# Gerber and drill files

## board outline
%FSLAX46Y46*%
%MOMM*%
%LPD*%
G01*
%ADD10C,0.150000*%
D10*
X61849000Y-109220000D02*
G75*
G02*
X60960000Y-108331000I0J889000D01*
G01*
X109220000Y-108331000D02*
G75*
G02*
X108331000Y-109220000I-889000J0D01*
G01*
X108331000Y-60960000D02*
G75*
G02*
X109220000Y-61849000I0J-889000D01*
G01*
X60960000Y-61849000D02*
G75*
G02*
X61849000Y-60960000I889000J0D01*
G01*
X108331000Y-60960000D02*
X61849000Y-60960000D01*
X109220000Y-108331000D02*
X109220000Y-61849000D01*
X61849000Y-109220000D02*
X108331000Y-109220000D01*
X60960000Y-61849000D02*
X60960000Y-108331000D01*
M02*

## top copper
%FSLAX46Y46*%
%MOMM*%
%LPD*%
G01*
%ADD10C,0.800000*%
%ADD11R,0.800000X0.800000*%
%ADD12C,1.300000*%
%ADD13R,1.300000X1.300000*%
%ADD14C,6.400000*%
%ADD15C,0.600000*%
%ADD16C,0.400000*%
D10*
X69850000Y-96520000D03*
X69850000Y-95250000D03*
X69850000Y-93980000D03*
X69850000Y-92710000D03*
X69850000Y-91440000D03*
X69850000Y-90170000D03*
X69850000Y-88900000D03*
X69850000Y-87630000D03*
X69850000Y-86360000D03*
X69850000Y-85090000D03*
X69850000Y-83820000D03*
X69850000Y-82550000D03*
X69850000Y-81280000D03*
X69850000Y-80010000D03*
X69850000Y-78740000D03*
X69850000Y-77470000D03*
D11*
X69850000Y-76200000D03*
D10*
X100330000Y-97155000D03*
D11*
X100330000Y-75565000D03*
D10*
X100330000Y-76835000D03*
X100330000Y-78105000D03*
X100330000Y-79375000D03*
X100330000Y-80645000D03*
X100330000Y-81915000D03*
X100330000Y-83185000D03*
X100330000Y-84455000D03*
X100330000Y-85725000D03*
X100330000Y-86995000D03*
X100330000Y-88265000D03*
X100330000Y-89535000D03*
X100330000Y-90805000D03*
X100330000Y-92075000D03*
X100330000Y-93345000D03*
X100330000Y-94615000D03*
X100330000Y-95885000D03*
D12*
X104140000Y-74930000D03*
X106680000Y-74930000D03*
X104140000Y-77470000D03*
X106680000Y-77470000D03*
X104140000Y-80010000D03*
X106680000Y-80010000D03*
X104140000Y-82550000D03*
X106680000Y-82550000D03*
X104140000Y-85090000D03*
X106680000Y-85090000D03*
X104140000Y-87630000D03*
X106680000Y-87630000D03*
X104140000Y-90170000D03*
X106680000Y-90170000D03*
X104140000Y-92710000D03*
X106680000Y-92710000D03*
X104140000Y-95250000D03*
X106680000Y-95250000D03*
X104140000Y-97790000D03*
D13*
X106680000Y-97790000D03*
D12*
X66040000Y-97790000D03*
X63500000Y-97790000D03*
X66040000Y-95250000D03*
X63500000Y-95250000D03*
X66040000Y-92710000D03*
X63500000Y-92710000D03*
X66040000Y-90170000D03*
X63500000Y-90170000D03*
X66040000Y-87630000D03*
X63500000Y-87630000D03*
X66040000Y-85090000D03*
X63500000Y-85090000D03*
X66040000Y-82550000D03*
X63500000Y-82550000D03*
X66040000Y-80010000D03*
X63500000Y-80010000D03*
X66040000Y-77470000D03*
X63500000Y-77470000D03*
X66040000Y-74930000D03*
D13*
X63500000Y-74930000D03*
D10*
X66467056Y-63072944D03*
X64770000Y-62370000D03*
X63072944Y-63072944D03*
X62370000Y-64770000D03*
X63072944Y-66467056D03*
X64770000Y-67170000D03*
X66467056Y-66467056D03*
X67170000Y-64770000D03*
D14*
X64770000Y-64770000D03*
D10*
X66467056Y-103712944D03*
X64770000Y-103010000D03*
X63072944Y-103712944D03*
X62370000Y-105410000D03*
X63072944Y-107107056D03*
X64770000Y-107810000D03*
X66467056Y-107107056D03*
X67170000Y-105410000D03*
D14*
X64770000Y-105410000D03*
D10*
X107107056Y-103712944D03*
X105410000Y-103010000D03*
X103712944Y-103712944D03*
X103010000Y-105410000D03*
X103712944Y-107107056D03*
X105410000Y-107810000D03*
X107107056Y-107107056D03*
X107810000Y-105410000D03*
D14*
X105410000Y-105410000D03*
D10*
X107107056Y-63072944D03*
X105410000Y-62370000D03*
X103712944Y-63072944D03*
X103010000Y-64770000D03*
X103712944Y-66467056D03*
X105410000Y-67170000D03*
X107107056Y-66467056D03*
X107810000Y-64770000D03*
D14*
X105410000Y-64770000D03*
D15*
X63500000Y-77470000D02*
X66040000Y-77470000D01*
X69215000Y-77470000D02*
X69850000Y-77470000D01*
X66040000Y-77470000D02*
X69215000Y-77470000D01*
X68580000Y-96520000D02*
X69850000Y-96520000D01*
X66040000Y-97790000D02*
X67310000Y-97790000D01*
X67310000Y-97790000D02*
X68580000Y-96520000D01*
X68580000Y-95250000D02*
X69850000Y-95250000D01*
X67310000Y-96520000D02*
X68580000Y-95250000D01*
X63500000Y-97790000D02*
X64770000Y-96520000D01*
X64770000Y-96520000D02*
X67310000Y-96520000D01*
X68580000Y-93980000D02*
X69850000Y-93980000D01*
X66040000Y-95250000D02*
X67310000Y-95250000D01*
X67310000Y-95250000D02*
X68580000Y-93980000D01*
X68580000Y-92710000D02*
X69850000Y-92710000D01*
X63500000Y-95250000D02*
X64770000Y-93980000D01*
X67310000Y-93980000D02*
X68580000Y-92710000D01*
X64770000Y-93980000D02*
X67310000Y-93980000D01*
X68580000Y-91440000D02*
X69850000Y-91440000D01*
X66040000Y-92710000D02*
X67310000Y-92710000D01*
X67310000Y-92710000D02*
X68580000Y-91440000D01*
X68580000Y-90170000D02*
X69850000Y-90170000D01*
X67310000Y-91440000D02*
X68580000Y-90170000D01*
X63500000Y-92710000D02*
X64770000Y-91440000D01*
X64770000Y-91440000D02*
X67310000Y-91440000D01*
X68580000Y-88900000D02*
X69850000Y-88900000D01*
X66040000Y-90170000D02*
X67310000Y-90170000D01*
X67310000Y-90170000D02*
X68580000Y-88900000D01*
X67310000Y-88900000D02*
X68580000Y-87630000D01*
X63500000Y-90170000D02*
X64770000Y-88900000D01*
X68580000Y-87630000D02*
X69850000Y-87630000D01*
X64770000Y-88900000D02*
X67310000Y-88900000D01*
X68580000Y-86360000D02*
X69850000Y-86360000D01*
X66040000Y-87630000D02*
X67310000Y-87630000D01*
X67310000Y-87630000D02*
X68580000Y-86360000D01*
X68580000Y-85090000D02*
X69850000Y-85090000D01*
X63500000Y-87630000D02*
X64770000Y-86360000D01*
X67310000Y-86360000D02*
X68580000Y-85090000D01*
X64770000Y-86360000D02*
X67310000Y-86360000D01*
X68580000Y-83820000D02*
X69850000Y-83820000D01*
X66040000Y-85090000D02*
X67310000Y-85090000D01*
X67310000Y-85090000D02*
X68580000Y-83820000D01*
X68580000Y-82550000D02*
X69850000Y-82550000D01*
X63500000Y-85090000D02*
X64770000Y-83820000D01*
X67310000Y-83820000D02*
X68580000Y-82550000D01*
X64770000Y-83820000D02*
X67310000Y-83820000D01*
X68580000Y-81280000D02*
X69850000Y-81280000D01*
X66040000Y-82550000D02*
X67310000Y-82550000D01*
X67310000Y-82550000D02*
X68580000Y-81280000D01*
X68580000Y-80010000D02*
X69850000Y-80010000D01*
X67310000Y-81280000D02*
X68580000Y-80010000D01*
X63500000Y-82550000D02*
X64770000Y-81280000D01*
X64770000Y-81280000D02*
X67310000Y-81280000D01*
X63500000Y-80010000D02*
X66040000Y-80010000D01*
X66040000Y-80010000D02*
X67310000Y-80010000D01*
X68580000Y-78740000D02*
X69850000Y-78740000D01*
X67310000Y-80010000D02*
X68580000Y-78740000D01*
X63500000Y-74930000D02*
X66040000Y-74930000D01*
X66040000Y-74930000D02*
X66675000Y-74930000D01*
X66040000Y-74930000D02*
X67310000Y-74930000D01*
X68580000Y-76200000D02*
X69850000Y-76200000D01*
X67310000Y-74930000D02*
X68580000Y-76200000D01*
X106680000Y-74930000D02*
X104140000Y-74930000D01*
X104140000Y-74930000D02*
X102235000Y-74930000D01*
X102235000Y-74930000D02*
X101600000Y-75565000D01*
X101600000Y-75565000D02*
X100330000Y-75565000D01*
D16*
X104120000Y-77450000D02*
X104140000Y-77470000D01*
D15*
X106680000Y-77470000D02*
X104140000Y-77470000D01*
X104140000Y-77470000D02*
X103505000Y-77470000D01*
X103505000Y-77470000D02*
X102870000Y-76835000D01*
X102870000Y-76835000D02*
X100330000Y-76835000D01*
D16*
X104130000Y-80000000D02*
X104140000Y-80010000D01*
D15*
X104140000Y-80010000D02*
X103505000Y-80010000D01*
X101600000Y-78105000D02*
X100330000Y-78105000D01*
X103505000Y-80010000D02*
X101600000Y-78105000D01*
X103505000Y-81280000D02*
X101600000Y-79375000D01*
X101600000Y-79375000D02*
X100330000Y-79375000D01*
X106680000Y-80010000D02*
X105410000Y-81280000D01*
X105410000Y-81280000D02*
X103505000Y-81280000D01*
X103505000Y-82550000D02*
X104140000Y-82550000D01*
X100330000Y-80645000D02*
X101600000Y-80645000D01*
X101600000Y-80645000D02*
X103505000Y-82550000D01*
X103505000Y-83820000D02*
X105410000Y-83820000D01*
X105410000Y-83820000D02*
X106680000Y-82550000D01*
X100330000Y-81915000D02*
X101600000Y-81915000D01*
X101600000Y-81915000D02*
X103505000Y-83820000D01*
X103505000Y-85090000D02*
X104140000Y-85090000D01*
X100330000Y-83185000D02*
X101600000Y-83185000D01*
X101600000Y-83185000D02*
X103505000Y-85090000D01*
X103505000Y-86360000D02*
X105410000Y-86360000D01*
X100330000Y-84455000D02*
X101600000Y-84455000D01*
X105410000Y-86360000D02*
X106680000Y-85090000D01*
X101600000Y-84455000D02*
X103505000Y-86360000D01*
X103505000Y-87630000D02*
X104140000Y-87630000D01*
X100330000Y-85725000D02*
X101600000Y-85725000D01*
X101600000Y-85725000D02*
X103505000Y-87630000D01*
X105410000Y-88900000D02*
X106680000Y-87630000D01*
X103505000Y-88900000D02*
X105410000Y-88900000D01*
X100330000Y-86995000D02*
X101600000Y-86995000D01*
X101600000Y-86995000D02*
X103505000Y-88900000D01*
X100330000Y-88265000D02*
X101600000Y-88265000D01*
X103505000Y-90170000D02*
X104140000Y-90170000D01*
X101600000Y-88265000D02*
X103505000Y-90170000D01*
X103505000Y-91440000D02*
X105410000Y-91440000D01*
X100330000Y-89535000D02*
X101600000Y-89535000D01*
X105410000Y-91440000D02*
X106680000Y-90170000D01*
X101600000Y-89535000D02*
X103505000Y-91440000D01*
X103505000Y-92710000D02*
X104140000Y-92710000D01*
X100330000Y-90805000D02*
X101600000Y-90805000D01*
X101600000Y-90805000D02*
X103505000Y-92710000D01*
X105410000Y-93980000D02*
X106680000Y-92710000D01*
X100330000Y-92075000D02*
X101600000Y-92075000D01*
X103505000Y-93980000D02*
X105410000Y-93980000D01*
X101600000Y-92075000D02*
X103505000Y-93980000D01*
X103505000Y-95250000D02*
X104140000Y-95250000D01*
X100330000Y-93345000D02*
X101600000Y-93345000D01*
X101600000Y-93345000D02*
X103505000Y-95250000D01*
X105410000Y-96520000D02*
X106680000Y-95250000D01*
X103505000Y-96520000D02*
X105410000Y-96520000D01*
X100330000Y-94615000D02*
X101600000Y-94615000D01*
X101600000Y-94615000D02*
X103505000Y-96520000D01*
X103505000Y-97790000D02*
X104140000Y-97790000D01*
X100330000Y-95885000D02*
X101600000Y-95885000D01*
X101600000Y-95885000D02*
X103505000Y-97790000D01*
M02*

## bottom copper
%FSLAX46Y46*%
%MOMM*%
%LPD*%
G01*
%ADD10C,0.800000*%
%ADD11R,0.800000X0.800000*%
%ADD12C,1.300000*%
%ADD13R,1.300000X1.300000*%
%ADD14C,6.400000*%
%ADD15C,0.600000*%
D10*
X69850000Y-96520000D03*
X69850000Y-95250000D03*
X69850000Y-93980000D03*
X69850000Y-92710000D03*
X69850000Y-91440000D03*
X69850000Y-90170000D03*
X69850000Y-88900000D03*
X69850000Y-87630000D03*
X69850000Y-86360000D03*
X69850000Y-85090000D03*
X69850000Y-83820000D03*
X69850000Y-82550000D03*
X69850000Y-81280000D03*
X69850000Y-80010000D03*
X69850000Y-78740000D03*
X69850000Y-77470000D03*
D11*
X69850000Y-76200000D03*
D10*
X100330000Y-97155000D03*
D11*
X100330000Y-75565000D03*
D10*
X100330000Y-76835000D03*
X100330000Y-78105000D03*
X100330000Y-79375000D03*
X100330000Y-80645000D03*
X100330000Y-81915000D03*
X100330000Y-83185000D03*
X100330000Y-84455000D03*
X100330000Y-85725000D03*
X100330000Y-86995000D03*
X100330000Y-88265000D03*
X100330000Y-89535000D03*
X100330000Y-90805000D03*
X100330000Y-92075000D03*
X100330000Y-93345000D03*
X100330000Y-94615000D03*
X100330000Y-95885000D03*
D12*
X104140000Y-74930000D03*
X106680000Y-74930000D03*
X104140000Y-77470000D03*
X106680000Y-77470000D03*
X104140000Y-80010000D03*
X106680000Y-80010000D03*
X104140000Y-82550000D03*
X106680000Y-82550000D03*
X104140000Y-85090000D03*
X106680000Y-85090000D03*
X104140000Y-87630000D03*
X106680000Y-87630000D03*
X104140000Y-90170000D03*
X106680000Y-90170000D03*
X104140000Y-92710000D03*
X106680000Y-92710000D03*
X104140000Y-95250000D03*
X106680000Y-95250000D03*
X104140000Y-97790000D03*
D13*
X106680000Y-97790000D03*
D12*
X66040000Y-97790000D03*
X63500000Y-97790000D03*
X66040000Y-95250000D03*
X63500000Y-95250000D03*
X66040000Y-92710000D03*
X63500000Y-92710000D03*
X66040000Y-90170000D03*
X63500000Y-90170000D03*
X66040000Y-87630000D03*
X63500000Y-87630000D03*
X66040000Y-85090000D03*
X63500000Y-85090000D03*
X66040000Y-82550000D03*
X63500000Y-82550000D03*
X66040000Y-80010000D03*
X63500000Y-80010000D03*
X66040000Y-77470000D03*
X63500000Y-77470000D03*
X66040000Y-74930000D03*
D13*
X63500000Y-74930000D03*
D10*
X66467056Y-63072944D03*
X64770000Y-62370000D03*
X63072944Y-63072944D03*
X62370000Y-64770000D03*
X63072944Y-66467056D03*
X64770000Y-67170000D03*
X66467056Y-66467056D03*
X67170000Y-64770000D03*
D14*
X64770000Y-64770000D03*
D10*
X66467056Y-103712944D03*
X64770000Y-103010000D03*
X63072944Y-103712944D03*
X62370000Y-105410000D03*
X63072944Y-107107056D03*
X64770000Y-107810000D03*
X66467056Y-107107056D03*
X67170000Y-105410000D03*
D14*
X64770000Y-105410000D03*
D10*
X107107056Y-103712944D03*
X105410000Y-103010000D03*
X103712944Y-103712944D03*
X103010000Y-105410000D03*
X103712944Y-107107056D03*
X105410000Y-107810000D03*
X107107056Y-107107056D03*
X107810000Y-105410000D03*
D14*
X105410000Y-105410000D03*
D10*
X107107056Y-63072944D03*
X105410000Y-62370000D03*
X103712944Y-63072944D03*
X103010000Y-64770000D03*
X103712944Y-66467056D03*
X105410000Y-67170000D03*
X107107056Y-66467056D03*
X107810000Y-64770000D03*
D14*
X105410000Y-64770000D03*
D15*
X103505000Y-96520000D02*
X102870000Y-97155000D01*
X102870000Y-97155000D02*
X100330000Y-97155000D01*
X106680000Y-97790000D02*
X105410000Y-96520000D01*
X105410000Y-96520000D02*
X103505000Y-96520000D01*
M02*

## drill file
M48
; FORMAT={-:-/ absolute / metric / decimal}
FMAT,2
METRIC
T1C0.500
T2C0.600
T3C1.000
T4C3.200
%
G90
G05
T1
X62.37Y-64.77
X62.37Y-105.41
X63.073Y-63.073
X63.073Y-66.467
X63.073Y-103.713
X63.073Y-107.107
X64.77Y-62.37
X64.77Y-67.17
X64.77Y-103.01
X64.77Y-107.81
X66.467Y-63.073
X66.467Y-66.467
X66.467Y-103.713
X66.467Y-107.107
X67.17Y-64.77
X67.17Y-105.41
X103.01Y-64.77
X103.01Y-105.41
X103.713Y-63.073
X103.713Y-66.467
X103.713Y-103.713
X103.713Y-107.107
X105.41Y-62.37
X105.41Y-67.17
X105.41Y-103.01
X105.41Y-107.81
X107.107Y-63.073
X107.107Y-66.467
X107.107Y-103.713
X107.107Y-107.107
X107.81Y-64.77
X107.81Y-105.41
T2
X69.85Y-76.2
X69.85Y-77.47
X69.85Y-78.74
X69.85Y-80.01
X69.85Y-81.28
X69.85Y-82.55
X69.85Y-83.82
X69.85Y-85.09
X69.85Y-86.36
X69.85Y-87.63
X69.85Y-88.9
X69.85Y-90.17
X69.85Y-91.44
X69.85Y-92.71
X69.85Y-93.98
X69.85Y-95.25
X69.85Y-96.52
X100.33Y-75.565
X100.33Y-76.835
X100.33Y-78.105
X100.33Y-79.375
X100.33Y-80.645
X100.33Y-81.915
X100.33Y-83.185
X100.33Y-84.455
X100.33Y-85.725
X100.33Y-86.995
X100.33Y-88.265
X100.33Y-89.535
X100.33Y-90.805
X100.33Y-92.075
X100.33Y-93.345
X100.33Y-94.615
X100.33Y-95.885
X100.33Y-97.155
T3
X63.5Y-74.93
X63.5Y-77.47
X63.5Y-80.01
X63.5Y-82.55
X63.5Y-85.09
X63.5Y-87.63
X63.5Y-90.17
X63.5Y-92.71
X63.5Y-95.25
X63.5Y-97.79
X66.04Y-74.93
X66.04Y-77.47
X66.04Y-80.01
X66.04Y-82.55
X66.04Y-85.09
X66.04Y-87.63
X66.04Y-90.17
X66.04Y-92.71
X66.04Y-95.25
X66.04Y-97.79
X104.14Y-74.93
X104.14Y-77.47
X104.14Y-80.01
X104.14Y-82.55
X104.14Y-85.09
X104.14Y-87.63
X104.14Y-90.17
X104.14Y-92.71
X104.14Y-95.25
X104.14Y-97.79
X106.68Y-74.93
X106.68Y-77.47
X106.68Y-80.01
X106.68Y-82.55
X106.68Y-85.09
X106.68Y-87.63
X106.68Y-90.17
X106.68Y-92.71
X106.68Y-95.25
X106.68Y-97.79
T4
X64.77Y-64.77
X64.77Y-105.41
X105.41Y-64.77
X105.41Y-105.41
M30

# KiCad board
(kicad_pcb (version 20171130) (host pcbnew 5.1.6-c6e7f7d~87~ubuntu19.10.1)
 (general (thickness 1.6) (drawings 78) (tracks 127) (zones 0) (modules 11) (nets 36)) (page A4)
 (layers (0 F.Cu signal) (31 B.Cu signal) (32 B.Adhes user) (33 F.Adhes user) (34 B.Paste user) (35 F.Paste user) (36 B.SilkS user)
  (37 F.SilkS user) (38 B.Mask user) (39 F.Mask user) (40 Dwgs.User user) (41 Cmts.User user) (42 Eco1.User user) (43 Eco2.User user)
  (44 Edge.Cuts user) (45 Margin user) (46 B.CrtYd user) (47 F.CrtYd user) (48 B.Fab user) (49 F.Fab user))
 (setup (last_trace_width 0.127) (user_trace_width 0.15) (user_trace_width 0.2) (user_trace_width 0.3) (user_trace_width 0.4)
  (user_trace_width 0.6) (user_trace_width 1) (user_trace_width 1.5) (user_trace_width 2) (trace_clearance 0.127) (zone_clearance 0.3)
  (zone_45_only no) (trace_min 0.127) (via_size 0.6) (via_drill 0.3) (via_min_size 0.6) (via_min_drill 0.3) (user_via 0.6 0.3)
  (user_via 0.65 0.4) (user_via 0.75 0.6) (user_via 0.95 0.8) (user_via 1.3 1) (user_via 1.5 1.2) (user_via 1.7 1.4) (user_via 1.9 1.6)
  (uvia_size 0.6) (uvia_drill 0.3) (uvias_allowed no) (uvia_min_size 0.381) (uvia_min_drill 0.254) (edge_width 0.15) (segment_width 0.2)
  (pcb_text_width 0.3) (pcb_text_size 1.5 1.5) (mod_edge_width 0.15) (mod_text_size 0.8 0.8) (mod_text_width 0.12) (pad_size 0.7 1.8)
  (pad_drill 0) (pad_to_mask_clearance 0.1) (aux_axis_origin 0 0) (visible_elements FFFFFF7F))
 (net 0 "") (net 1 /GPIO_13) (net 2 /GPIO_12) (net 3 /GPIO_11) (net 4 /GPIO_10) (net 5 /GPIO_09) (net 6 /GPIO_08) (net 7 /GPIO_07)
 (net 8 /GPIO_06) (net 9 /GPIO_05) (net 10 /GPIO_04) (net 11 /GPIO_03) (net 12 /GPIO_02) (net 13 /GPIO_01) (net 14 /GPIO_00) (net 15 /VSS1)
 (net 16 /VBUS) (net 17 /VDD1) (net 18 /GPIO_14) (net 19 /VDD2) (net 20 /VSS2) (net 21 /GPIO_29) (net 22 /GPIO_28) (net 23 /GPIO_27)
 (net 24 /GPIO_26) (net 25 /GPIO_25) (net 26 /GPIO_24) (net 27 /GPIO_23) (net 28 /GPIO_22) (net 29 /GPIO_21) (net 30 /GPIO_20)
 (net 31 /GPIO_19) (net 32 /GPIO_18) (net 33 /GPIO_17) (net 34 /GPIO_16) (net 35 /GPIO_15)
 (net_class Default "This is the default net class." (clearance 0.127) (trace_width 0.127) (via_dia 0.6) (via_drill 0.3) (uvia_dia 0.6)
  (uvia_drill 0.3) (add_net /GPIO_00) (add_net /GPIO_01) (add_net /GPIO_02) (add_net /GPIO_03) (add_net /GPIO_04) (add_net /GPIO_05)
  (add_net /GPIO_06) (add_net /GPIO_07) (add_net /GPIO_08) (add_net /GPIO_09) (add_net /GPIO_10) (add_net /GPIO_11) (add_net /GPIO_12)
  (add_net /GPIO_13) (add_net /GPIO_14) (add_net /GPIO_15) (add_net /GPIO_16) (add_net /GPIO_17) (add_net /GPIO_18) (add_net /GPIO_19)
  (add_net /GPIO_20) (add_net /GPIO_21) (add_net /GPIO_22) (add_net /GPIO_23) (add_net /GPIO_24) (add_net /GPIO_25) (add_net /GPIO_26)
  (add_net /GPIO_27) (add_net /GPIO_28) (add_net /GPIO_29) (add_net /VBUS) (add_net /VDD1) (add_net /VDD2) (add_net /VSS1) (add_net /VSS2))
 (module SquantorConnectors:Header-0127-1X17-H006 (layer F.Cu) (at 69.85 86.36 270)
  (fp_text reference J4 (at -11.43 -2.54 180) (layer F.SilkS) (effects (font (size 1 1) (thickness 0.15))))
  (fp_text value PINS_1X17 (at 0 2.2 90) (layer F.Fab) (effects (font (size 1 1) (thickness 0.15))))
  (pad 17 thru_hole circle (at 10.16 0 270) (size 0.8 0.8) (drill 0.6) (layers *.Cu *.Mask) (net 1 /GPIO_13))
  (pad 16 thru_hole circle (at 8.89 0 270) (size 0.8 0.8) (drill 0.6) (layers *.Cu *.Mask) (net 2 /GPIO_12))
  (pad 15 thru_hole circle (at 7.62 0 270) (size 0.8 0.8) (drill 0.6) (layers *.Cu *.Mask) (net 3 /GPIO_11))
  (pad 14 thru_hole circle (at 6.35 0 270) (size 0.8 0.8) (drill 0.6) (layers *.Cu *.Mask) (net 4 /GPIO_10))
  (pad 13 thru_hole circle (at 5.08 0 270) (size 0.8 0.8) (drill 0.6) (layers *.Cu *.Mask) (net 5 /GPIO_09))
  (pad 12 thru_hole circle (at 3.81 0 270) (size 0.8 0.8) (drill 0.6) (layers *.Cu *.Mask) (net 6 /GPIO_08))
  (pad 11 thru_hole circle (at 2.54 0 270) (size 0.8 0.8) (drill 0.6) (layers *.Cu *.Mask) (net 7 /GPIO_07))
  (pad 10 thru_hole circle (at 1.27 0 270) (size 0.8 0.8) (drill 0.6) (layers *.Cu *.Mask) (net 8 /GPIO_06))
  (pad 9 thru_hole circle (at 0 0 270) (size 0.8 0.8) (drill 0.6) (layers *.Cu *.Mask) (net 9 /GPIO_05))
  (pad 8 thru_hole circle (at -1.27 0 270) (size 0.8 0.8) (drill 0.6) (layers *.Cu *.Mask) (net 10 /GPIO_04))
  (pad 7 thru_hole circle (at -2.54 0 270) (size 0.8 0.8) (drill 0.6) (layers *.Cu *.Mask) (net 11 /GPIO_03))
  (pad 6 thru_hole circle (at -3.81 0 270) (size 0.8 0.8) (drill 0.6) (layers *.Cu *.Mask) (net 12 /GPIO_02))
  (pad 5 thru_hole circle (at -5.08 0 270) (size 0.8 0.8) (drill 0.6) (layers *.Cu *.Mask) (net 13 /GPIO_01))
  (pad 4 thru_hole circle (at -6.35 0 270) (size 0.8 0.8) (drill 0.6) (layers *.Cu *.Mask) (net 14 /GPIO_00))
  (pad 3 thru_hole circle (at -7.62 0 270) (size 0.8 0.8) (drill 0.6) (layers *.Cu *.Mask) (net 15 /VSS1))
  (pad 2 thru_hole circle (at -8.89 0 270) (size 0.8 0.8) (drill 0.6) (layers *.Cu *.Mask) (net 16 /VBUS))
  (pad 1 thru_hole rect (at -10.16 0 270) (size 0.8 0.8) (drill 0.6) (layers *.Cu *.Mask) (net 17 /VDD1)))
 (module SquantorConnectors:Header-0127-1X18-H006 (layer F.Cu) (at 100.33 86.36 270)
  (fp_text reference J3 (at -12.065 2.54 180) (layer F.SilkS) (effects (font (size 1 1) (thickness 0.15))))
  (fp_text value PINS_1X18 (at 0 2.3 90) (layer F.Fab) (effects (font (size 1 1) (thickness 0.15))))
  (pad 18 thru_hole circle (at 10.795 0 270) (size 0.8 0.8) (drill 0.6) (layers *.Cu *.Mask) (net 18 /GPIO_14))
  (pad 1 thru_hole rect (at -10.795 0 270) (size 0.8 0.8) (drill 0.6) (layers *.Cu *.Mask) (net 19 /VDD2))
  (pad 2 thru_hole circle (at -9.525 0 270) (size 0.8 0.8) (drill 0.6) (layers *.Cu *.Mask) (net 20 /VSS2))
  (pad 3 thru_hole circle (at -8.255 0 270) (size 0.8 0.8) (drill 0.6) (layers *.Cu *.Mask) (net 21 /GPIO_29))
  (pad 4 thru_hole circle (at -6.985 0 270) (size 0.8 0.8) (drill 0.6) (layers *.Cu *.Mask) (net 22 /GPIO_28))
  (pad 5 thru_hole circle (at -5.715 0 270) (size 0.8 0.8) (drill 0.6) (layers *.Cu *.Mask) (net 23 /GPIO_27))
  (pad 6 thru_hole circle (at -4.445 0 270) (size 0.8 0.8) (drill 0.6) (layers *.Cu *.Mask) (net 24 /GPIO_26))
  (pad 7 thru_hole circle (at -3.175 0 270) (size 0.8 0.8) (drill 0.6) (layers *.Cu *.Mask) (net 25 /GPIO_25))
  (pad 8 thru_hole circle (at -1.905 0 270) (size 0.8 0.8) (drill 0.6) (layers *.Cu *.Mask) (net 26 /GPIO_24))
  (pad 9 thru_hole circle (at -0.635 0 270) (size 0.8 0.8) (drill 0.6) (layers *.Cu *.Mask) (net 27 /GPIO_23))
  (pad 10 thru_hole circle (at 0.635 0 270) (size 0.8 0.8) (drill 0.6) (layers *.Cu *.Mask) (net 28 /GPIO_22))
  (pad 11 thru_hole circle (at 1.905 0 270) (size 0.8 0.8) (drill 0.6) (layers *.Cu *.Mask) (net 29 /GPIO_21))
  (pad 12 thru_hole circle (at 3.175 0 270) (size 0.8 0.8) (drill 0.6) (layers *.Cu *.Mask) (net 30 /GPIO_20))
  (pad 13 thru_hole circle (at 4.445 0 270) (size 0.8 0.8) (drill 0.6) (layers *.Cu *.Mask) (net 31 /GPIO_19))
  (pad 14 thru_hole circle (at 5.715 0 270) (size 0.8 0.8) (drill 0.6) (layers *.Cu *.Mask) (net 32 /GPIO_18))
  (pad 15 thru_hole circle (at 6.985 0 270) (size 0.8 0.8) (drill 0.6) (layers *.Cu *.Mask) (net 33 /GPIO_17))
  (pad 16 thru_hole circle (at 8.255 0 270) (size 0.8 0.8) (drill 0.6) (layers *.Cu *.Mask) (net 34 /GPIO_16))
  (pad 17 thru_hole circle (at 9.525 0 270) (size 0.8 0.8) (drill 0.6) (layers *.Cu *.Mask) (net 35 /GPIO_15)))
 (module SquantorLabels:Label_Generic (layer B.Cu) (at 83.7 105.9)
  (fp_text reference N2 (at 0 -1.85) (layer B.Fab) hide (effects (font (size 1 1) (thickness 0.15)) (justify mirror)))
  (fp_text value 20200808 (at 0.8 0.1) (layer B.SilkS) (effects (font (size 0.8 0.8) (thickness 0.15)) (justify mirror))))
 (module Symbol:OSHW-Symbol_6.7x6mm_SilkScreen (layer B.Cu) (at 85.2 101.9 180)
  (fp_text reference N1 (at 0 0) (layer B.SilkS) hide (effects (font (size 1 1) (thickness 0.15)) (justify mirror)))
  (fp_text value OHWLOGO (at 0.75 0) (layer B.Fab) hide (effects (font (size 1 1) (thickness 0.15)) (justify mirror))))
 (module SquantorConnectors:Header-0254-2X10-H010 (layer F.Cu) (at 105.41 86.36 90)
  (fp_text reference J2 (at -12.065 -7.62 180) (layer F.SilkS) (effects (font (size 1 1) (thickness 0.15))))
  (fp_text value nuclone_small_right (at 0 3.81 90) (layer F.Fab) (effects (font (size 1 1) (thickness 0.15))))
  (pad 20 thru_hole circle (at 11.43 -1.27 90) (size 1.3 1.3) (drill 1) (layers *.Cu *.Mask) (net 19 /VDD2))
  (pad 19 thru_hole circle (at 11.43 1.27 90) (size 1.3 1.3) (drill 1) (layers *.Cu *.Mask) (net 19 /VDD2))
  (pad 18 thru_hole circle (at 8.89 -1.27 90) (size 1.3 1.3) (drill 1) (layers *.Cu *.Mask) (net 20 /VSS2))
  (pad 17 thru_hole circle (at 8.89 1.27 90) (size 1.3 1.3) (drill 1) (layers *.Cu *.Mask) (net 20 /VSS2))
  (pad 16 thru_hole circle (at 6.35 -1.27 90) (size 1.3 1.3) (drill 1) (layers *.Cu *.Mask) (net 21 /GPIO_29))
  (pad 15 thru_hole circle (at 6.35 1.27 90) (size 1.3 1.3) (drill 1) (layers *.Cu *.Mask) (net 22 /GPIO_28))
  (pad 14 thru_hole circle (at 3.81 -1.27 90) (size 1.3 1.3) (drill 1) (layers *.Cu *.Mask) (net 23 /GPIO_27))
  (pad 13 thru_hole circle (at 3.81 1.27 90) (size 1.3 1.3) (drill 1) (layers *.Cu *.Mask) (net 24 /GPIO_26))
  (pad 12 thru_hole circle (at 1.27 -1.27 90) (size 1.3 1.3) (drill 1) (layers *.Cu *.Mask) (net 25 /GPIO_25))
  (pad 11 thru_hole circle (at 1.27 1.27 90) (size 1.3 1.3) (drill 1) (layers *.Cu *.Mask) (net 26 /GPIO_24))
  (pad 10 thru_hole circle (at -1.27 -1.27 90) (size 1.3 1.3) (drill 1) (layers *.Cu *.Mask) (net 27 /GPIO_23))
  (pad 9 thru_hole circle (at -1.27 1.27 90) (size 1.3 1.3) (drill 1) (layers *.Cu *.Mask) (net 28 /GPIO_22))
  (pad 8 thru_hole circle (at -3.81 -1.27 90) (size 1.3 1.3) (drill 1) (layers *.Cu *.Mask) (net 29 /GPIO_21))
  (pad 7 thru_hole circle (at -3.81 1.27 90) (size 1.3 1.3) (drill 1) (layers *.Cu *.Mask) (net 30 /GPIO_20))
  (pad 6 thru_hole circle (at -6.35 -1.27 90) (size 1.3 1.3) (drill 1) (layers *.Cu *.Mask) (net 31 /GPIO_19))
  (pad 5 thru_hole circle (at -6.35 1.27 90) (size 1.3 1.3) (drill 1) (layers *.Cu *.Mask) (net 32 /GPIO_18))
  (pad 4 thru_hole circle (at -8.89 -1.27 90) (size 1.3 1.3) (drill 1) (layers *.Cu *.Mask) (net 33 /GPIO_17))
  (pad 3 thru_hole circle (at -8.89 1.27 90) (size 1.3 1.3) (drill 1) (layers *.Cu *.Mask) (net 34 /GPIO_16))
  (pad 2 thru_hole circle (at -11.43 -1.27 90) (size 1.3 1.3) (drill 1) (layers *.Cu *.Mask) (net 35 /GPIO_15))
  (pad 1 thru_hole rect (at -11.43 1.27 90) (size 1.3 1.3) (drill 1) (layers *.Cu *.Mask) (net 18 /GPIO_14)))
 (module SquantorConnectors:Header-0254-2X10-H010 (layer F.Cu) (at 64.77 86.36 270)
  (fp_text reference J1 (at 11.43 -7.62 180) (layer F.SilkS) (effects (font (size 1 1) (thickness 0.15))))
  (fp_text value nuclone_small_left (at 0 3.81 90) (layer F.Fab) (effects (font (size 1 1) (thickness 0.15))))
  (pad 20 thru_hole circle (at 11.43 -1.27 270) (size 1.3 1.3) (drill 1) (layers *.Cu *.Mask) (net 1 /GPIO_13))
  (pad 19 thru_hole circle (at 11.43 1.27 270) (size 1.3 1.3) (drill 1) (layers *.Cu *.Mask) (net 2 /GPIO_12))
  (pad 18 thru_hole circle (at 8.89 -1.27 270) (size 1.3 1.3) (drill 1) (layers *.Cu *.Mask) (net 3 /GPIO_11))
  (pad 17 thru_hole circle (at 8.89 1.27 270) (size 1.3 1.3) (drill 1) (layers *.Cu *.Mask) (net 4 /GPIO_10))
  (pad 16 thru_hole circle (at 6.35 -1.27 270) (size 1.3 1.3) (drill 1) (layers *.Cu *.Mask) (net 5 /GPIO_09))
  (pad 15 thru_hole circle (at 6.35 1.27 270) (size 1.3 1.3) (drill 1) (layers *.Cu *.Mask) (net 6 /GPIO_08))
  (pad 14 thru_hole circle (at 3.81 -1.27 270) (size 1.3 1.3) (drill 1) (layers *.Cu *.Mask) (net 7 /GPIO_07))
  (pad 13 thru_hole circle (at 3.81 1.27 270) (size 1.3 1.3) (drill 1) (layers *.Cu *.Mask) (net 8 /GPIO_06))
  (pad 12 thru_hole circle (at 1.27 -1.27 270) (size 1.3 1.3) (drill 1) (layers *.Cu *.Mask) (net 9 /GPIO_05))
  (pad 11 thru_hole circle (at 1.27 1.27 270) (size 1.3 1.3) (drill 1) (layers *.Cu *.Mask) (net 10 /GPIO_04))
  (pad 10 thru_hole circle (at -1.27 -1.27 270) (size 1.3 1.3) (drill 1) (layers *.Cu *.Mask) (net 11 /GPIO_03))
  (pad 9 thru_hole circle (at -1.27 1.27 270) (size 1.3 1.3) (drill 1) (layers *.Cu *.Mask) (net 12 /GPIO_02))
  (pad 8 thru_hole circle (at -3.81 -1.27 270) (size 1.3 1.3) (drill 1) (layers *.Cu *.Mask) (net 13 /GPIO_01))
  (pad 7 thru_hole circle (at -3.81 1.27 270) (size 1.3 1.3) (drill 1) (layers *.Cu *.Mask) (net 14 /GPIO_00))
  (pad 6 thru_hole circle (at -6.35 -1.27 270) (size 1.3 1.3) (drill 1) (layers *.Cu *.Mask) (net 15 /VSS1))
  (pad 5 thru_hole circle (at -6.35 1.27 270) (size 1.3 1.3) (drill 1) (layers *.Cu *.Mask) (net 15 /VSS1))
  (pad 4 thru_hole circle (at -8.89 -1.27 270) (size 1.3 1.3) (drill 1) (layers *.Cu *.Mask) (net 16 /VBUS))
  (pad 3 thru_hole circle (at -8.89 1.27 270) (size 1.3 1.3) (drill 1) (layers *.Cu *.Mask) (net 16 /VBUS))
  (pad 2 thru_hole circle (at -11.43 -1.27 270) (size 1.3 1.3) (drill 1) (layers *.Cu *.Mask) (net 17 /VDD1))
  (pad 1 thru_hole rect (at -11.43 1.27 270) (size 1.3 1.3) (drill 1) (layers *.Cu *.Mask) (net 17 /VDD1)))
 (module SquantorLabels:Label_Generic (layer B.Cu) (at 86 107.9 180)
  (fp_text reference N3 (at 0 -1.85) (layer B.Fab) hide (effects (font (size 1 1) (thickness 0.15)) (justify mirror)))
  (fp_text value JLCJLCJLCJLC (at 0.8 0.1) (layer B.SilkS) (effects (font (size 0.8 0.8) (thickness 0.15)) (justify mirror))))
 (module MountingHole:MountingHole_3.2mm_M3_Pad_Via (layer F.Cu) (at 64.77 64.77)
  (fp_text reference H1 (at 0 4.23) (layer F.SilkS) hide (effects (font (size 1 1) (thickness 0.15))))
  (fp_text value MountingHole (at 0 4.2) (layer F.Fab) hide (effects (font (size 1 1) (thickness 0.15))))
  (pad 1 thru_hole circle (at 1.697056 -1.697056) (size 0.8 0.8) (drill 0.5) (layers *.Cu *.Mask))
  (pad 1 thru_hole circle (at 0 -2.4) (size 0.8 0.8) (drill 0.5) (layers *.Cu *.Mask))
  (pad 1 thru_hole circle (at -1.697056 -1.697056) (size 0.8 0.8) (drill 0.5) (layers *.Cu *.Mask))
  (pad 1 thru_hole circle (at -2.4 0) (size 0.8 0.8) (drill 0.5) (layers *.Cu *.Mask))
  (pad 1 thru_hole circle (at -1.697056 1.697056) (size 0.8 0.8) (drill 0.5) (layers *.Cu *.Mask))
  (pad 1 thru_hole circle (at 0 2.4) (size 0.8 0.8) (drill 0.5) (layers *.Cu *.Mask))
  (pad 1 thru_hole circle (at 1.697056 1.697056) (size 0.8 0.8) (drill 0.5) (layers *.Cu *.Mask))
  (pad 1 thru_hole circle (at 2.4 0) (size 0.8 0.8) (drill 0.5) (layers *.Cu *.Mask))
  (pad 1 thru_hole circle (at 0 0) (size 6.4 6.4) (drill 3.2) (layers *.Cu *.Mask)))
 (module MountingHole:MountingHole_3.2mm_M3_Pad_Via (layer F.Cu) (at 64.77 105.41)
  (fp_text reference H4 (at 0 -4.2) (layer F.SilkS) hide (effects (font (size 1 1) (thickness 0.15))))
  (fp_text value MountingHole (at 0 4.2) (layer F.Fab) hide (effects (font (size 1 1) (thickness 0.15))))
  (pad 1 thru_hole circle (at 1.697056 -1.697056) (size 0.8 0.8) (drill 0.5) (layers *.Cu *.Mask))
  (pad 1 thru_hole circle (at 0 -2.4) (size 0.8 0.8) (drill 0.5) (layers *.Cu *.Mask))
  (pad 1 thru_hole circle (at -1.697056 -1.697056) (size 0.8 0.8) (drill 0.5) (layers *.Cu *.Mask))
  (pad 1 thru_hole circle (at -2.4 0) (size 0.8 0.8) (drill 0.5) (layers *.Cu *.Mask))
  (pad 1 thru_hole circle (at -1.697056 1.697056) (size 0.8 0.8) (drill 0.5) (layers *.Cu *.Mask))
  (pad 1 thru_hole circle (at 0 2.4) (size 0.8 0.8) (drill 0.5) (layers *.Cu *.Mask))
  (pad 1 thru_hole circle (at 1.697056 1.697056) (size 0.8 0.8) (drill 0.5) (layers *.Cu *.Mask))
  (pad 1 thru_hole circle (at 2.4 0) (size 0.8 0.8) (drill 0.5) (layers *.Cu *.Mask))
  (pad 1 thru_hole circle (at 0 0) (size 6.4 6.4) (drill 3.2) (layers *.Cu *.Mask)))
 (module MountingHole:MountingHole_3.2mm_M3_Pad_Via (layer F.Cu) (at 105.41 105.41)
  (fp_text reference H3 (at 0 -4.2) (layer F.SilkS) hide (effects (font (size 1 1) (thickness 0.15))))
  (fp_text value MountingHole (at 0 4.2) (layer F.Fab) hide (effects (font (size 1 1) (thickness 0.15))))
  (pad 1 thru_hole circle (at 1.697056 -1.697056) (size 0.8 0.8) (drill 0.5) (layers *.Cu *.Mask))
  (pad 1 thru_hole circle (at 0 -2.4) (size 0.8 0.8) (drill 0.5) (layers *.Cu *.Mask))
  (pad 1 thru_hole circle (at -1.697056 -1.697056) (size 0.8 0.8) (drill 0.5) (layers *.Cu *.Mask))
  (pad 1 thru_hole circle (at -2.4 0) (size 0.8 0.8) (drill 0.5) (layers *.Cu *.Mask))
  (pad 1 thru_hole circle (at -1.697056 1.697056) (size 0.8 0.8) (drill 0.5) (layers *.Cu *.Mask))
  (pad 1 thru_hole circle (at 0 2.4) (size 0.8 0.8) (drill 0.5) (layers *.Cu *.Mask))
  (pad 1 thru_hole circle (at 1.697056 1.697056) (size 0.8 0.8) (drill 0.5) (layers *.Cu *.Mask))
  (pad 1 thru_hole circle (at 2.4 0) (size 0.8 0.8) (drill 0.5) (layers *.Cu *.Mask))
  (pad 1 thru_hole circle (at 0 0) (size 6.4 6.4) (drill 3.2) (layers *.Cu *.Mask)))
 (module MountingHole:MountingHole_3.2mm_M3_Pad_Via (layer F.Cu) (at 105.41 64.77)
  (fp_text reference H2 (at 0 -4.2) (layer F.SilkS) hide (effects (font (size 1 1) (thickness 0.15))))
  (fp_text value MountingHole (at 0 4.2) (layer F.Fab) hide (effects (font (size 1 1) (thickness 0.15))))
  (pad 1 thru_hole circle (at 1.697056 -1.697056) (size 0.8 0.8) (drill 0.5) (layers *.Cu *.Mask))
  (pad 1 thru_hole circle (at 0 -2.4) (size 0.8 0.8) (drill 0.5) (layers *.Cu *.Mask))
  (pad 1 thru_hole circle (at -1.697056 -1.697056) (size 0.8 0.8) (drill 0.5) (layers *.Cu *.Mask))
  (pad 1 thru_hole circle (at -2.4 0) (size 0.8 0.8) (drill 0.5) (layers *.Cu *.Mask))
  (pad 1 thru_hole circle (at -1.697056 1.697056) (size 0.8 0.8) (drill 0.5) (layers *.Cu *.Mask))
  (pad 1 thru_hole circle (at 0 2.4) (size 0.8 0.8) (drill 0.5) (layers *.Cu *.Mask))
  (pad 1 thru_hole circle (at 1.697056 1.697056) (size 0.8 0.8) (drill 0.5) (layers *.Cu *.Mask))
  (pad 1 thru_hole circle (at 2.4 0) (size 0.8 0.8) (drill 0.5) (layers *.Cu *.Mask))
  (pad 1 thru_hole circle (at 0 0) (size 6.4 6.4) (drill 3.2) (layers *.Cu *.Mask)))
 (gr_arc (start 61.849 108.331) (end 60.96 108.331) (angle -90) (layer Edge.Cuts) (width 0.15))
 (gr_arc (start 108.331 108.331) (end 108.331 109.22) (angle -90) (layer Edge.Cuts) (width 0.15))
 (gr_arc (start 108.331 61.849) (end 109.22 61.849) (angle -90) (layer Edge.Cuts) (width 0.15))
 (gr_arc (start 61.849 61.849) (end 61.849 60.96) (angle -90) (layer Edge.Cuts) (width 0.15))
 (gr_line (start 108.331 60.96) (end 61.849 60.96) (layer Edge.Cuts) (width 0.15))
 (gr_line (start 109.22 108.331) (end 109.22 61.849) (layer Edge.Cuts) (width 0.15))
 (gr_line (start 61.849 109.22) (end 108.331 109.22) (layer Edge.Cuts) (width 0.15))
 (gr_line (start 60.96 61.849) (end 60.96 108.331) (layer Edge.Cuts) (width 0.15))
 (segment (start 63.5 77.47) (end 66.04 77.47) (width 0.6) (layer F.Cu) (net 16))
 (segment (start 69.215 77.47) (end 69.85 77.47) (width 0.6) (layer F.Cu) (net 16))
 (segment (start 66.04 77.47) (end 69.215 77.47) (width 0.6) (layer F.Cu) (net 16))
 (segment (start 68.58 96.52) (end 69.85 96.52) (width 0.6) (layer F.Cu) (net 1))
 (segment (start 66.04 97.79) (end 67.31 97.79) (width 0.6) (layer F.Cu) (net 1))
 (segment (start 67.31 97.79) (end 68.58 96.52) (width 0.6) (layer F.Cu) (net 1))
 (segment (start 68.58 95.25) (end 69.85 95.25) (width 0.6) (layer F.Cu) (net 2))
 (segment (start 67.31 96.52) (end 68.58 95.25) (width 0.6) (layer F.Cu) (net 2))
 (segment (start 63.5 97.79) (end 64.77 96.52) (width 0.6) (layer F.Cu) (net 2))
 (segment (start 64.77 96.52) (end 67.31 96.52) (width 0.6) (layer F.Cu) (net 2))
 (segment (start 68.58 93.98) (end 69.85 93.98) (width 0.6) (layer F.Cu) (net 3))
 (segment (start 66.04 95.25) (end 67.31 95.25) (width 0.6) (layer F.Cu) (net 3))
 (segment (start 67.31 95.25) (end 68.58 93.98) (width 0.6) (layer F.Cu) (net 3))
 (segment (start 68.58 92.71) (end 69.85 92.71) (width 0.6) (layer F.Cu) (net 4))
 (segment (start 63.5 95.25) (end 64.77 93.98) (width 0.6) (layer F.Cu) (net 4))
 (segment (start 67.31 93.98) (end 68.58 92.71) (width 0.6) (layer F.Cu) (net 4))
 (segment (start 64.77 93.98) (end 67.31 93.98) (width 0.6) (layer F.Cu) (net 4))
 (segment (start 68.58 91.44) (end 69.85 91.44) (width 0.6) (layer F.Cu) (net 5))
 (segment (start 66.04 92.71) (end 67.31 92.71) (width 0.6) (layer F.Cu) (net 5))
 (segment (start 67.31 92.71) (end 68.58 91.44) (width 0.6) (layer F.Cu) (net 5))
 (segment (start 68.58 90.17) (end 69.85 90.17) (width 0.6) (layer F.Cu) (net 6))
 (segment (start 67.31 91.44) (end 68.58 90.17) (width 0.6) (layer F.Cu) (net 6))
 (segment (start 63.5 92.71) (end 64.77 91.44) (width 0.6) (layer F.Cu) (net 6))
 (segment (start 64.77 91.44) (end 67.31 91.44) (width 0.6) (layer F.Cu) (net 6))
 (segment (start 68.58 88.9) (end 69.85 88.9) (width 0.6) (layer F.Cu) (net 7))
 (segment (start 66.04 90.17) (end 67.31 90.17) (width 0.6) (layer F.Cu) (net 7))
 (segment (start 67.31 90.17) (end 68.58 88.9) (width 0.6) (layer F.Cu) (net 7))
 (segment (start 67.31 88.9) (end 68.58 87.63) (width 0.6) (layer F.Cu) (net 8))
 (segment (start 63.5 90.17) (end 64.77 88.9) (width 0.6) (layer F.Cu) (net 8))
 (segment (start 68.58 87.63) (end 69.85 87.63) (width 0.6) (layer F.Cu) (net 8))
 (segment (start 64.77 88.9) (end 67.31 88.9) (width 0.6) (layer F.Cu) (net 8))
 (segment (start 68.58 86.36) (end 69.85 86.36) (width 0.6) (layer F.Cu) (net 9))
 (segment (start 66.04 87.63) (end 67.31 87.63) (width 0.6) (layer F.Cu) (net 9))
 (segment (start 67.31 87.63) (end 68.58 86.36) (width 0.6) (layer F.Cu) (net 9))
 (segment (start 68.58 85.09) (end 69.85 85.09) (width 0.6) (layer F.Cu) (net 10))
 (segment (start 63.5 87.63) (end 64.77 86.36) (width 0.6) (layer F.Cu) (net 10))
 (segment (start 67.31 86.36) (end 68.58 85.09) (width 0.6) (layer F.Cu) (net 10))
 (segment (start 64.77 86.36) (end 67.31 86.36) (width 0.6) (layer F.Cu) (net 10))
 (segment (start 68.58 83.82) (end 69.85 83.82) (width 0.6) (layer F.Cu) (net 11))
 (segment (start 66.04 85.09) (end 67.31 85.09) (width 0.6) (layer F.Cu) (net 11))
 (segment (start 67.31 85.09) (end 68.58 83.82) (width 0.6) (layer F.Cu) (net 11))
 (segment (start 68.58 82.55) (end 69.85 82.55) (width 0.6) (layer F.Cu) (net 12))
 (segment (start 63.5 85.09) (end 64.77 83.82) (width 0.6) (layer F.Cu) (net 12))
 (segment (start 67.31 83.82) (end 68.58 82.55) (width 0.6) (layer F.Cu) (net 12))
 (segment (start 64.77 83.82) (end 67.31 83.82) (width 0.6) (layer F.Cu) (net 12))
 (segment (start 68.58 81.28) (end 69.85 81.28) (width 0.6) (layer F.Cu) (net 13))
 (segment (start 66.04 82.55) (end 67.31 82.55) (width 0.6) (layer F.Cu) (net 13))
 (segment (start 67.31 82.55) (end 68.58 81.28) (width 0.6) (layer F.Cu) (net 13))
 (segment (start 68.58 80.01) (end 69.85 80.01) (width 0.6) (layer F.Cu) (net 14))
 (segment (start 67.31 81.28) (end 68.58 80.01) (width 0.6) (layer F.Cu) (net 14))
 (segment (start 63.5 82.55) (end 64.77 81.28) (width 0.6) (layer F.Cu) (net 14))
 (segment (start 64.77 81.28) (end 67.31 81.28) (width 0.6) (layer F.Cu) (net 14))
 (segment (start 63.5 80.01) (end 66.04 80.01) (width 0.6) (layer F.Cu) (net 15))
 (segment (start 66.04 80.01) (end 67.31 80.01) (width 0.6) (layer F.Cu) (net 15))
 (segment (start 68.58 78.74) (end 69.85 78.74) (width 0.6) (layer F.Cu) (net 15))
 (segment (start 67.31 80.01) (end 68.58 78.74) (width 0.6) (layer F.Cu) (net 15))
 (segment (start 63.5 74.93) (end 66.04 74.93) (width 0.6) (layer F.Cu) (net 17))
 (segment (start 66.04 74.93) (end 66.675 74.93) (width 0.6) (layer F.Cu) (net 17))
 (segment (start 66.04 74.93) (end 67.31 74.93) (width 0.6) (layer F.Cu) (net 17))
 (segment (start 68.58 76.2) (end 69.85 76.2) (width 0.6) (layer F.Cu) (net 17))
 (segment (start 67.31 74.93) (end 68.58 76.2) (width 0.6) (layer F.Cu) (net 17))
 (segment (start 106.68 74.93) (end 104.14 74.93) (width 0.6) (layer F.Cu) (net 19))
 (segment (start 104.14 74.93) (end 102.235 74.93) (width 0.6) (layer F.Cu) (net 19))
 (segment (start 102.235 74.93) (end 101.6 75.565) (width 0.6) (layer F.Cu) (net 19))
 (segment (start 101.6 75.565) (end 100.33 75.565) (width 0.6) (layer F.Cu) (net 19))
 (segment (start 104.12 77.45) (end 104.14 77.47) (width 0.4) (layer F.Cu) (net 20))
 (segment (start 106.68 77.47) (end 104.14 77.47) (width 0.6) (layer F.Cu) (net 20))
 (segment (start 104.14 77.47) (end 103.505 77.47) (width 0.6) (layer F.Cu) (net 20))
 (segment (start 103.505 77.47) (end 102.87 76.835) (width 0.6) (layer F.Cu) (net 20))
 (segment (start 102.87 76.835) (end 100.33 76.835) (width 0.6) (layer F.Cu) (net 20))
 (segment (start 104.13 80) (end 104.14 80.01) (width 0.4) (layer F.Cu) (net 21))
 (segment (start 104.14 80.01) (end 103.505 80.01) (width 0.6) (layer F.Cu) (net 21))
 (segment (start 101.6 78.105) (end 100.33 78.105) (width 0.6) (layer F.Cu) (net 21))
 (segment (start 103.505 80.01) (end 101.6 78.105) (width 0.6) (layer F.Cu) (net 21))
 (segment (start 103.505 81.28) (end 101.6 79.375) (width 0.6) (layer F.Cu) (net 22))
 (segment (start 101.6 79.375) (end 100.33 79.375) (width 0.6) (layer F.Cu) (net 22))
 (segment (start 106.68 80.01) (end 105.41 81.28) (width 0.6) (layer F.Cu) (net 22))
 (segment (start 105.41 81.28) (end 103.505 81.28) (width 0.6) (layer F.Cu) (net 22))
 (segment (start 103.505 82.55) (end 104.14 82.55) (width 0.6) (layer F.Cu) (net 23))
 (segment (start 100.33 80.645) (end 101.6 80.645) (width 0.6) (layer F.Cu) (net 23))
 (segment (start 101.6 80.645) (end 103.505 82.55) (width 0.6) (layer F.Cu) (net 23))
 (segment (start 103.505 83.82) (end 105.41 83.82) (width 0.6) (layer F.Cu) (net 24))
 (segment (start 105.41 83.82) (end 106.68 82.55) (width 0.6) (layer F.Cu) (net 24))
 (segment (start 100.33 81.915) (end 101.6 81.915) (width 0.6) (layer F.Cu) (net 24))
 (segment (start 101.6 81.915) (end 103.505 83.82) (width 0.6) (layer F.Cu) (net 24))
 (segment (start 103.505 85.09) (end 104.14 85.09) (width 0.6) (layer F.Cu) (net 25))
 (segment (start 100.33 83.185) (end 101.6 83.185) (width 0.6) (layer F.Cu) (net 25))
 (segment (start 101.6 83.185) (end 103.505 85.09) (width 0.6) (layer F.Cu) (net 25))
 (segment (start 103.505 86.36) (end 105.41 86.36) (width 0.6) (layer F.Cu) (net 26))
 (segment (start 100.33 84.455) (end 101.6 84.455) (width 0.6) (layer F.Cu) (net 26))
 (segment (start 105.41 86.36) (end 106.68 85.09) (width 0.6) (layer F.Cu) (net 26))
 (segment (start 101.6 84.455) (end 103.505 86.36) (width 0.6) (layer F.Cu) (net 26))
 (segment (start 103.505 87.63) (end 104.14 87.63) (width 0.6) (layer F.Cu) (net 27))
 (segment (start 100.33 85.725) (end 101.6 85.725) (width 0.6) (layer F.Cu) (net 27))
 (segment (start 101.6 85.725) (end 103.505 87.63) (width 0.6) (layer F.Cu) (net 27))
 (segment (start 105.41 88.9) (end 106.68 87.63) (width 0.6) (layer F.Cu) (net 28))
 (segment (start 103.505 88.9) (end 105.41 88.9) (width 0.6) (layer F.Cu) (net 28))
 (segment (start 100.33 86.995) (end 101.6 86.995) (width 0.6) (layer F.Cu) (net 28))
 (segment (start 101.6 86.995) (end 103.505 88.9) (width 0.6) (layer F.Cu) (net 28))
 (segment (start 100.33 88.265) (end 101.6 88.265) (width 0.6) (layer F.Cu) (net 29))
 (segment (start 103.505 90.17) (end 104.14 90.17) (width 0.6) (layer F.Cu) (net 29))
 (segment (start 101.6 88.265) (end 103.505 90.17) (width 0.6) (layer F.Cu) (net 29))
 (segment (start 103.505 91.44) (end 105.41 91.44) (width 0.6) (layer F.Cu) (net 30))
 (segment (start 100.33 89.535) (end 101.6 89.535) (width 0.6) (layer F.Cu) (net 30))
 (segment (start 105.41 91.44) (end 106.68 90.17) (width 0.6) (layer F.Cu) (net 30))
 (segment (start 101.6 89.535) (end 103.505 91.44) (width 0.6) (layer F.Cu) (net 30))
 (segment (start 103.505 92.71) (end 104.14 92.71) (width 0.6) (layer F.Cu) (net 31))
 (segment (start 100.33 90.805) (end 101.6 90.805) (width 0.6) (layer F.Cu) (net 31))
 (segment (start 101.6 90.805) (end 103.505 92.71) (width 0.6) (layer F.Cu) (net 31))
 (segment (start 105.41 93.98) (end 106.68 92.71) (width 0.6) (layer F.Cu) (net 32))
 (segment (start 100.33 92.075) (end 101.6 92.075) (width 0.6) (layer F.Cu) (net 32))
 (segment (start 103.505 93.98) (end 105.41 93.98) (width 0.6) (layer F.Cu) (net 32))
 (segment (start 101.6 92.075) (end 103.505 93.98) (width 0.6) (layer F.Cu) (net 32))
 (segment (start 103.505 95.25) (end 104.14 95.25) (width 0.6) (layer F.Cu) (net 33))
 (segment (start 100.33 93.345) (end 101.6 93.345) (width 0.6) (layer F.Cu) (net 33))
 (segment (start 101.6 93.345) (end 103.505 95.25) (width 0.6) (layer F.Cu) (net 33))
 (segment (start 105.41 96.52) (end 106.68 95.25) (width 0.6) (layer F.Cu) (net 34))
 (segment (start 103.505 96.52) (end 105.41 96.52) (width 0.6) (layer F.Cu) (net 34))
 (segment (start 100.33 94.615) (end 101.6 94.615) (width 0.6) (layer F.Cu) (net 34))
 (segment (start 101.6 94.615) (end 103.505 96.52) (width 0.6) (layer F.Cu) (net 34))
 (segment (start 103.505 97.79) (end 104.14 97.79) (width 0.6) (layer F.Cu) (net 35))
 (segment (start 100.33 95.885) (end 101.6 95.885) (width 0.6) (layer F.Cu) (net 35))
 (segment (start 101.6 95.885) (end 103.505 97.79) (width 0.6) (layer F.Cu) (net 35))
 (segment (start 103.505 96.52) (end 102.87 97.155) (width 0.6) (layer B.Cu) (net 18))
 (segment (start 102.87 97.155) (end 100.33 97.155) (width 0.6) (layer B.Cu) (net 18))
 (segment (start 106.68 97.79) (end 105.41 96.52) (width 0.6) (layer B.Cu) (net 18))
 (segment (start 105.41 96.52) (end 103.505 96.52) (width 0.6) (layer B.Cu) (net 18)))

